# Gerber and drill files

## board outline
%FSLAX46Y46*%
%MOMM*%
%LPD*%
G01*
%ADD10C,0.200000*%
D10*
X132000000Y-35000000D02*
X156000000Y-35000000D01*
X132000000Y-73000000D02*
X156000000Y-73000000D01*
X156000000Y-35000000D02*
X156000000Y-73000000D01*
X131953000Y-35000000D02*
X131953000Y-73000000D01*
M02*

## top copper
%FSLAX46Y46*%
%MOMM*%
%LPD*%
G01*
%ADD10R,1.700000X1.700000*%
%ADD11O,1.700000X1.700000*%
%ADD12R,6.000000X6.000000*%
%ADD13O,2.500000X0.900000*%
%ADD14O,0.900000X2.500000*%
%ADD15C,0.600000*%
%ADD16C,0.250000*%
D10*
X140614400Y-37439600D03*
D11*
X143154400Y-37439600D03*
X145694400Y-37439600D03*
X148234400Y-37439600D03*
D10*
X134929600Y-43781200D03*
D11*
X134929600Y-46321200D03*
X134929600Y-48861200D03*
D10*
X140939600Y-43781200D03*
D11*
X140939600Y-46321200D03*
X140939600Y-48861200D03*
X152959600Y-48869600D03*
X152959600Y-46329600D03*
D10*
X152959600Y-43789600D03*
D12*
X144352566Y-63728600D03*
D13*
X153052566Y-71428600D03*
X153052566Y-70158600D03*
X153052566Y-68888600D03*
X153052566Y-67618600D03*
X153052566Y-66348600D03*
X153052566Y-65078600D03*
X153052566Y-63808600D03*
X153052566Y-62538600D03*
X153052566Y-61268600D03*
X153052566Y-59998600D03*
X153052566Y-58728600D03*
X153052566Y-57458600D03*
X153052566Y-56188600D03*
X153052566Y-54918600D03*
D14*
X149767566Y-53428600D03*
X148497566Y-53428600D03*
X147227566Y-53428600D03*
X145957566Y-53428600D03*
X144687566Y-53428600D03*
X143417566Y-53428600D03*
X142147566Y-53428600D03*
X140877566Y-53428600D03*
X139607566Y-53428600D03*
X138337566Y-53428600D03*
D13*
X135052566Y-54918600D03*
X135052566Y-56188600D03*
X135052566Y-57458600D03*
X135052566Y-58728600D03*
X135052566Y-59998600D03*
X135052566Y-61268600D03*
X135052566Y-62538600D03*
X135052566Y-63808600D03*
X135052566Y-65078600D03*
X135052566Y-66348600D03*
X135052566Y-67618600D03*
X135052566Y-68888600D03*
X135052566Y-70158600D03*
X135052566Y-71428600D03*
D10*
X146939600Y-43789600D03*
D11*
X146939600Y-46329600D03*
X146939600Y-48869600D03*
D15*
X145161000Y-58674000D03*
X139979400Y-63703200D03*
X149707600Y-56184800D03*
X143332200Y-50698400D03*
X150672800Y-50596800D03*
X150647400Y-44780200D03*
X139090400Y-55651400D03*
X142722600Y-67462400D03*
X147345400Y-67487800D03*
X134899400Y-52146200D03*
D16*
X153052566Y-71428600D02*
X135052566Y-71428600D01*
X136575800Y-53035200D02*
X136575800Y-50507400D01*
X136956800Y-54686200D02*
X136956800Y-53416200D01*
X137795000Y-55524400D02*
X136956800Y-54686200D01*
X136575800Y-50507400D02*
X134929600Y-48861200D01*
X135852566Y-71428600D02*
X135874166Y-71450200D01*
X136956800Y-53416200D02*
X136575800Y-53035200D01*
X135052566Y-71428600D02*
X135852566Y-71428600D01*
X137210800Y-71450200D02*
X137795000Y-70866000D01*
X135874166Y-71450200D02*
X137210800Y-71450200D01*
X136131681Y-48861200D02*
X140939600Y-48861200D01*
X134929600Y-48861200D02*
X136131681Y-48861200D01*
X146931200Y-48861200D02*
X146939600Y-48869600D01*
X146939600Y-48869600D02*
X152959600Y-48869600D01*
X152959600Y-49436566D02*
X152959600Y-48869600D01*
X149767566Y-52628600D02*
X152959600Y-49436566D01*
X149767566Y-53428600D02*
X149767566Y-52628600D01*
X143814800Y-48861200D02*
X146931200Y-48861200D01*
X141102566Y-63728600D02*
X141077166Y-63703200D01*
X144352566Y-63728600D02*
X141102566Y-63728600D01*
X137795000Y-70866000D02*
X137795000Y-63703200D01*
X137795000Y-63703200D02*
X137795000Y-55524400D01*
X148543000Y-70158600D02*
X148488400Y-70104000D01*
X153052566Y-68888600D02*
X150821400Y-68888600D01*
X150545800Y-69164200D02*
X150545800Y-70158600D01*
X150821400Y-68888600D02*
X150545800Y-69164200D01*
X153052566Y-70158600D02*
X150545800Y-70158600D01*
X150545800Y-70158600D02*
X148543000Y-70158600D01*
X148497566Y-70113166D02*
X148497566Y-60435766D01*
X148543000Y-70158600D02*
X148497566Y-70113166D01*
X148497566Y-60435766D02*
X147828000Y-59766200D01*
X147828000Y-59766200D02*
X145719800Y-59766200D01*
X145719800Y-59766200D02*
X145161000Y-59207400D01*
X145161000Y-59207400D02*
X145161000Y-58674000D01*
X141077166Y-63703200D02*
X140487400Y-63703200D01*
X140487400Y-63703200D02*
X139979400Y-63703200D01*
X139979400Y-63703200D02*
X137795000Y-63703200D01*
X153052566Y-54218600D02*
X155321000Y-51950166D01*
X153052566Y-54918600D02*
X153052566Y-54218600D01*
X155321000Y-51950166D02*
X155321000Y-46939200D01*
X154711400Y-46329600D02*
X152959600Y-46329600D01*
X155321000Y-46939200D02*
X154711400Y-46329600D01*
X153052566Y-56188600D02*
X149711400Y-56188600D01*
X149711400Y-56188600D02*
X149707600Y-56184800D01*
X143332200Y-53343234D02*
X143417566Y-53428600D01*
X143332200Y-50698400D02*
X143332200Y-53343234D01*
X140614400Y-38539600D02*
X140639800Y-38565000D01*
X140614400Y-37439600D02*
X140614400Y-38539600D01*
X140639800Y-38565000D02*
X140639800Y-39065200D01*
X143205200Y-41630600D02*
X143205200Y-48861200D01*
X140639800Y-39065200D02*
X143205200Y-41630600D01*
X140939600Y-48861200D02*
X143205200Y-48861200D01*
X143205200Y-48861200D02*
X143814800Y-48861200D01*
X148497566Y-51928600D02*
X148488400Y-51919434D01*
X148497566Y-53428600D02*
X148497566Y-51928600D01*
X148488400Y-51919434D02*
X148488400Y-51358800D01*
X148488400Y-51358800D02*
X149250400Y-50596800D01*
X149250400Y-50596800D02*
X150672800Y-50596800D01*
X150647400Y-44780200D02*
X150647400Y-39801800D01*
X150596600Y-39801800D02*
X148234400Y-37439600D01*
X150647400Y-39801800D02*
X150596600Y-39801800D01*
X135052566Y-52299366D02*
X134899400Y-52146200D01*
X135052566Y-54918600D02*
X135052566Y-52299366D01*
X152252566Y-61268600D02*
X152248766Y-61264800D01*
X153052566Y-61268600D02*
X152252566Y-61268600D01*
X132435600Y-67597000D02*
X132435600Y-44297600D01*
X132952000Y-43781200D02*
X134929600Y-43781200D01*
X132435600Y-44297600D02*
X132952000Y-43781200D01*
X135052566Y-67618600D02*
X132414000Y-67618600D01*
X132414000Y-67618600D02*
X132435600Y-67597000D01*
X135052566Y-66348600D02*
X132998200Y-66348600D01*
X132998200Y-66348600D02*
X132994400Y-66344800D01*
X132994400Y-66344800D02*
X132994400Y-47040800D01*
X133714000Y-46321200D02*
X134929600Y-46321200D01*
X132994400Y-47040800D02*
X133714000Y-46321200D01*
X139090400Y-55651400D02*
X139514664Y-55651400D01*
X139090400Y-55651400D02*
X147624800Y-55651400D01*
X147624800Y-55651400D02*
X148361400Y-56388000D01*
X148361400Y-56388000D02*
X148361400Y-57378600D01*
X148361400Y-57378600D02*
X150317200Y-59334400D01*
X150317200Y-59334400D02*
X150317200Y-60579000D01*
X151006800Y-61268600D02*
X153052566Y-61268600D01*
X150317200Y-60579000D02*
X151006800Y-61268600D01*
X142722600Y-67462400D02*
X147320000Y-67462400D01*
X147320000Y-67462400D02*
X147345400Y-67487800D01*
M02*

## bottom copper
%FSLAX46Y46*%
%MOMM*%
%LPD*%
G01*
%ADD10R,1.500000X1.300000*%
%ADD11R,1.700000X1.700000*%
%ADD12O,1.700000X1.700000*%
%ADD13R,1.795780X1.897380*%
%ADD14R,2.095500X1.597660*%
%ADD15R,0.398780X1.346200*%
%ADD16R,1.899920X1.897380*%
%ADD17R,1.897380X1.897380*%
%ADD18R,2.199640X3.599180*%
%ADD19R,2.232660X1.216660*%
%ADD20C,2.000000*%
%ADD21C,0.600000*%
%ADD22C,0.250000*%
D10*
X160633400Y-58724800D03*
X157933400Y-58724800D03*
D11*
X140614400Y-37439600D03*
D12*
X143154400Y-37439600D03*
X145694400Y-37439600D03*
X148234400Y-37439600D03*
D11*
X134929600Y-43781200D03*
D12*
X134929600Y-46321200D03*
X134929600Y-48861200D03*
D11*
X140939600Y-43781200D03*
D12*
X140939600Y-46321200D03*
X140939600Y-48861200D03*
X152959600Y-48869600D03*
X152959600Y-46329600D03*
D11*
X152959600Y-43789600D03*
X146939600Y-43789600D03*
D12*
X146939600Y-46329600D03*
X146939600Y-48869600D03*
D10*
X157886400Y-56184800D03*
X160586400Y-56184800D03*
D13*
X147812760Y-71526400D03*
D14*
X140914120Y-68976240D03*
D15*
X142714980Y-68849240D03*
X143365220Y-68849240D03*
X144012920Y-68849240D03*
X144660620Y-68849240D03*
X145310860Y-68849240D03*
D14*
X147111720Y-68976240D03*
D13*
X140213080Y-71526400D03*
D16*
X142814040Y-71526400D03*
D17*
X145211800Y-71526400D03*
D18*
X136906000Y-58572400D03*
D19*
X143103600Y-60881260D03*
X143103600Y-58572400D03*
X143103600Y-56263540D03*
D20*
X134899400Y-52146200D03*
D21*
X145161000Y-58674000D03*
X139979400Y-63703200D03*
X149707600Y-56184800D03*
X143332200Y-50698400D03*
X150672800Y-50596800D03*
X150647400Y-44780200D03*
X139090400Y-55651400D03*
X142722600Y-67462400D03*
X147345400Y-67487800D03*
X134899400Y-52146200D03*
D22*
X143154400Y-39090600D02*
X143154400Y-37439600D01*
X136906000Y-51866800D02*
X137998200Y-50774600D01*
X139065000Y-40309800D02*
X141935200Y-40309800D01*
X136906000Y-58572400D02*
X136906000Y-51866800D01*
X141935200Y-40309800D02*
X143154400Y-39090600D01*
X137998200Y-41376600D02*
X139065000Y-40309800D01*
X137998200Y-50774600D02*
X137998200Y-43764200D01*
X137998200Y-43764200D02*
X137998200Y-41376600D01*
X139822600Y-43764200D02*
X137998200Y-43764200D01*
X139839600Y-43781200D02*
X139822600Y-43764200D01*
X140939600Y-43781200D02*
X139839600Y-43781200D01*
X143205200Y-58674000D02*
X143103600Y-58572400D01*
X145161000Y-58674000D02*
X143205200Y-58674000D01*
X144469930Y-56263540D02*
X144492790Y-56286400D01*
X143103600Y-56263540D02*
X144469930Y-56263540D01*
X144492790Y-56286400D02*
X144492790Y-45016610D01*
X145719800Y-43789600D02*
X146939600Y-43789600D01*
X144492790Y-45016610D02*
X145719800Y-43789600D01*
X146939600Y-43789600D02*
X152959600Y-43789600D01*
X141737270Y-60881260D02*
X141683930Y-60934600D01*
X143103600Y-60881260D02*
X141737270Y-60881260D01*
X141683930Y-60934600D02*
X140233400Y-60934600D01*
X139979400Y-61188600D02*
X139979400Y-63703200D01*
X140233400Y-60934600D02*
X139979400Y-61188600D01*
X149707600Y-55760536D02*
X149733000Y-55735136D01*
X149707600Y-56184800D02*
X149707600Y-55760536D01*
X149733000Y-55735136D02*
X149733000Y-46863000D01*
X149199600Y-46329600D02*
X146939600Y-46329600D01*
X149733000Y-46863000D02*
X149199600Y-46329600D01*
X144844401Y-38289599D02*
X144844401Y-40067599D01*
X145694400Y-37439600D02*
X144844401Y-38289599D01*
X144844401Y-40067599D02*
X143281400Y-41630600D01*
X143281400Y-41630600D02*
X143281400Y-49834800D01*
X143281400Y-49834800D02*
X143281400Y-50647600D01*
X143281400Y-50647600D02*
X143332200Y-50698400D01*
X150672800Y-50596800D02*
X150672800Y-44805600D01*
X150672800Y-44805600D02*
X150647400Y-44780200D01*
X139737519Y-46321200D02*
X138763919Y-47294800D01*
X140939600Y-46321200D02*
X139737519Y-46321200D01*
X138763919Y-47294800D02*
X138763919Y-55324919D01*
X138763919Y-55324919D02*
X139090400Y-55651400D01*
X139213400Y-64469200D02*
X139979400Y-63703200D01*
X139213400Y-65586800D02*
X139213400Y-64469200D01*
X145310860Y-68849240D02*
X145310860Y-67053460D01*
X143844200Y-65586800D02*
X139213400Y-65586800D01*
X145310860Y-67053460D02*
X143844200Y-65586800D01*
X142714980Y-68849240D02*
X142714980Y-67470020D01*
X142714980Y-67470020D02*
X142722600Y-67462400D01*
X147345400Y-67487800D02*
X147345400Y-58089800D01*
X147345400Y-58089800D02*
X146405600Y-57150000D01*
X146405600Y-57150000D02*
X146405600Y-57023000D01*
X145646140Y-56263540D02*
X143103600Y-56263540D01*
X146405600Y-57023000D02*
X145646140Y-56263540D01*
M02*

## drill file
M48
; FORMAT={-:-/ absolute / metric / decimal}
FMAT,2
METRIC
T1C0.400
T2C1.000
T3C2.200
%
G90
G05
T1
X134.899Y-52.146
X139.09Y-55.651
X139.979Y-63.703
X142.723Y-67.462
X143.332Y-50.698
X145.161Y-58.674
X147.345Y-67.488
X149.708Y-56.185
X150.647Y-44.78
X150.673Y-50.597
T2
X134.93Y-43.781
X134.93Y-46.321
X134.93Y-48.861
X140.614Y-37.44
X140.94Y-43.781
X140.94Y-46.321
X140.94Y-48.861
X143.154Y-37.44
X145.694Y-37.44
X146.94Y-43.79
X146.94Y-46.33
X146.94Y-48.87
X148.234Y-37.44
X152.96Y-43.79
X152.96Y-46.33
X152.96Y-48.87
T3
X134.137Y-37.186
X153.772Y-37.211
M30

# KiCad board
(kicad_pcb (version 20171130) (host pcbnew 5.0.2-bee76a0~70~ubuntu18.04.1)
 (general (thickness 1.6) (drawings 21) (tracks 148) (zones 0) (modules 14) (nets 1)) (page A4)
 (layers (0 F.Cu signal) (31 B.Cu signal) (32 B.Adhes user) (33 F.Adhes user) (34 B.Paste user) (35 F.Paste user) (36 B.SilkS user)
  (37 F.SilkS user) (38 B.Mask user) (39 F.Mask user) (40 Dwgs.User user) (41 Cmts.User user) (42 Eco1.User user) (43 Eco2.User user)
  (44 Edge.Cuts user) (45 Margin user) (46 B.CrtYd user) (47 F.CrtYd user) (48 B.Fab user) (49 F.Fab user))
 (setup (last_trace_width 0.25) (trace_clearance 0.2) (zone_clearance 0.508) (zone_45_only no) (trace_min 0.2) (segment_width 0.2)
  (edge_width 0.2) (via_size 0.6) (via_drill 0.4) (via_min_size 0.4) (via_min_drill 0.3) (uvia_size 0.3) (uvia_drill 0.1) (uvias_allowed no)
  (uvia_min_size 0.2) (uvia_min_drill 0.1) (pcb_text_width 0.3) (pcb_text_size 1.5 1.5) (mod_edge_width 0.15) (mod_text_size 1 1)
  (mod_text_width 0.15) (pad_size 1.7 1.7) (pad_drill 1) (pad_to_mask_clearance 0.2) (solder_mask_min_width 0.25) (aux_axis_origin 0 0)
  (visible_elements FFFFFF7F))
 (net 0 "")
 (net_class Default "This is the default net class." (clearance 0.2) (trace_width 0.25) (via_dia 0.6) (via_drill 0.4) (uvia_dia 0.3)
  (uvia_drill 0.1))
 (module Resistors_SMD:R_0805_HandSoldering (layer B.Cu) (at 159.2834 58.7248)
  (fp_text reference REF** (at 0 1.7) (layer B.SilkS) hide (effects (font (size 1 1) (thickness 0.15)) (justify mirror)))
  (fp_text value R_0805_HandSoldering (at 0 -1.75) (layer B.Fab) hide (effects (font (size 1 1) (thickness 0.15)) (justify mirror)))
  (pad 2 smd rect (at 1.35 0) (size 1.5 1.3) (layers B.Cu B.Paste B.Mask))
  (pad 1 smd rect (at -1.35 0) (size 1.5 1.3) (layers B.Cu B.Paste B.Mask)))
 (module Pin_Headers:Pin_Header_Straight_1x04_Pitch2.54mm (layer F.Cu) (at 140.6144 37.4396 90)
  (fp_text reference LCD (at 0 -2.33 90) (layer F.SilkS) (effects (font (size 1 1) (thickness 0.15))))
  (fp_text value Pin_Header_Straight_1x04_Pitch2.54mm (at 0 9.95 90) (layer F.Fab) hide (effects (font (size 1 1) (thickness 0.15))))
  (pad GND thru_hole rect (at 0 0 90) (size 1.7 1.7) (drill 1) (layers *.Cu *.Mask))
  (pad 3.3V thru_hole oval (at 0 2.54 90) (size 1.7 1.7) (drill 1) (layers *.Cu *.Mask))
  (pad CK thru_hole oval (at 0 5.08 90) (size 1.7 1.7) (drill 1) (layers *.Cu *.Mask))
  (pad DA thru_hole oval (at 0 7.62 90) (size 1.7 1.7) (drill 1) (layers *.Cu *.Mask)))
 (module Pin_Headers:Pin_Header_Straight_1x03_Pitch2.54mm (layer F.Cu) (at 134.9296 43.7812)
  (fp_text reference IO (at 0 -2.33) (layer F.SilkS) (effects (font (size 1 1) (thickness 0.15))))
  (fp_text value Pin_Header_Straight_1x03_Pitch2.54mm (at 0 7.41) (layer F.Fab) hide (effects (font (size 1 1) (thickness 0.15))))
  (pad TX thru_hole rect (at 0 0) (size 1.7 1.7) (drill 1) (layers *.Cu *.Mask))
  (pad RX thru_hole oval (at 0 2.54) (size 1.7 1.7) (drill 1) (layers *.Cu *.Mask))
  (pad 3 thru_hole oval (at 0 5.08) (size 1.7 1.7) (drill 1) (layers *.Cu *.Mask)))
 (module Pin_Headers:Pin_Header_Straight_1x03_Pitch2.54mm (layer F.Cu) (at 140.9396 43.7812)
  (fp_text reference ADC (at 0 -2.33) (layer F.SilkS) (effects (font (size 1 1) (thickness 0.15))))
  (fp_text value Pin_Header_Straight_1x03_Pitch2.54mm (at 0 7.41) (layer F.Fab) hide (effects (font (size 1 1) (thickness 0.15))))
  (pad +3.3v thru_hole rect (at 0 0) (size 1.7 1.7) (drill 1) (layers *.Cu *.Mask))
  (pad 2 thru_hole oval (at 0 2.54) (size 1.7 1.7) (drill 1) (layers *.Cu *.Mask))
  (pad 3 thru_hole oval (at 0 5.08) (size 1.7 1.7) (drill 1) (layers *.Cu *.Mask)))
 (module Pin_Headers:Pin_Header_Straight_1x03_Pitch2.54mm (layer F.Cu) (at 152.9596 43.7896)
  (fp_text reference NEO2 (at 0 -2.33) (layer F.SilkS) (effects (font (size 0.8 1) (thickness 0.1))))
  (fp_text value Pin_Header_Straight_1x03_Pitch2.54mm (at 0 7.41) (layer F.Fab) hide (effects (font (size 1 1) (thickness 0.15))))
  (pad GND thru_hole oval (at 0 5.08) (size 1.7 1.7) (drill 1) (layers *.Cu *.Mask))
  (pad 2 thru_hole oval (at 0 2.54) (size 1.7 1.7) (drill 1) (layers *.Cu *.Mask))
  (pad +V thru_hole rect (at 0 0) (size 1.7 1.7) (drill 1) (layers *.Cu *.Mask)))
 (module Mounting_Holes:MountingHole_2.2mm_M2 (layer F.Cu) (at 134.1374 37.1856)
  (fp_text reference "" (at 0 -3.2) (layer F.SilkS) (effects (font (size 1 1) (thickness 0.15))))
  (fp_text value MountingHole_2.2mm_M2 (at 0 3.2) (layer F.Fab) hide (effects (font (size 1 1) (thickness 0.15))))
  (pad 1 np_thru_hole circle (at 0 0) (size 2.2 2.2) (drill 2.2) (layers *.Cu *.Mask F.SilkS)))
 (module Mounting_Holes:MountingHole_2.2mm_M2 (layer F.Cu) (at 153.7716 37.211)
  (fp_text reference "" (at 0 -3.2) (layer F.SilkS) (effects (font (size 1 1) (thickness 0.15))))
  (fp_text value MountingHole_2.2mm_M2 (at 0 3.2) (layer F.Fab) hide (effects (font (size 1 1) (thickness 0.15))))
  (pad 1 np_thru_hole circle (at 0 0) (size 2.2 2.2) (drill 2.2) (layers *.Cu *.Mask F.SilkS)))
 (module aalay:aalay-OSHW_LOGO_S (layer B.Cu) (at 133.9596 40.259)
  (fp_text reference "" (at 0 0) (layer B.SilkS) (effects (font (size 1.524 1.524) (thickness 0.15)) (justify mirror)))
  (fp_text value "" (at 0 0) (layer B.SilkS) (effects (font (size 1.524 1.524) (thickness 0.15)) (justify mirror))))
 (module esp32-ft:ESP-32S (layer F.Cu) (at 144 61.911262 180)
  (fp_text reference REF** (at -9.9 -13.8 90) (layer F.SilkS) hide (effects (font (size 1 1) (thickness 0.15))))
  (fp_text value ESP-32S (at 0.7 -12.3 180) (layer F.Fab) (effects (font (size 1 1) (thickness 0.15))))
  (pad 39 smd rect (at -0.352566 -1.817338) (size 6 6) (layers F.Cu F.Paste F.Mask))
  (pad 1 smd oval (at -9.052566 -9.517338) (size 2.5 0.9) (layers F.Cu F.Paste F.Mask))
  (pad 2 smd oval (at -9.052566 -8.247338) (size 2.5 0.9) (layers F.Cu F.Paste F.Mask))
  (pad 3 smd oval (at -9.052566 -6.977338) (size 2.5 0.9) (layers F.Cu F.Paste F.Mask))
  (pad 4 smd oval (at -9.052566 -5.707338) (size 2.5 0.9) (layers F.Cu F.Paste F.Mask))
  (pad 5 smd oval (at -9.052566 -4.437338) (size 2.5 0.9) (layers F.Cu F.Paste F.Mask))
  (pad 6 smd oval (at -9.052566 -3.167338) (size 2.5 0.9) (layers F.Cu F.Paste F.Mask))
  (pad 7 smd oval (at -9.052566 -1.897338) (size 2.5 0.9) (layers F.Cu F.Paste F.Mask))
  (pad 8 smd oval (at -9.052566 -0.627338) (size 2.5 0.9) (layers F.Cu F.Paste F.Mask))
  (pad 9 smd oval (at -9.052566 0.642662) (size 2.5 0.9) (layers F.Cu F.Paste F.Mask))
  (pad 10 smd oval (at -9.052566 1.912662) (size 2.5 0.9) (layers F.Cu F.Paste F.Mask))
  (pad 11 smd oval (at -9.052566 3.182662) (size 2.5 0.9) (layers F.Cu F.Paste F.Mask))
  (pad 12 smd oval (at -9.052566 4.452662) (size 2.5 0.9) (layers F.Cu F.Paste F.Mask))
  (pad 13 smd oval (at -9.052566 5.722662) (size 2.5 0.9) (layers F.Cu F.Paste F.Mask))
  (pad 14 smd oval (at -9.052566 6.992662) (size 2.5 0.9) (layers F.Cu F.Paste F.Mask))
  (pad 15 smd oval (at -5.767566 8.482662) (size 0.9 2.5) (layers F.Cu F.Paste F.Mask))
  (pad 16 smd oval (at -4.497566 8.482662) (size 0.9 2.5) (layers F.Cu F.Paste F.Mask))
  (pad 17 smd oval (at -3.227566 8.482662) (size 0.9 2.5) (layers F.Cu F.Paste F.Mask))
  (pad 18 smd oval (at -1.957566 8.482662) (size 0.9 2.5) (layers F.Cu F.Paste F.Mask))
  (pad 19 smd oval (at -0.687566 8.482662) (size 0.9 2.5) (layers F.Cu F.Paste F.Mask))
  (pad 20 smd oval (at 0.582434 8.482662) (size 0.9 2.5) (layers F.Cu F.Paste F.Mask))
  (pad 21 smd oval (at 1.852434 8.482662) (size 0.9 2.5) (layers F.Cu F.Paste F.Mask))
  (pad 22 smd oval (at 3.122434 8.482662) (size 0.9 2.5) (layers F.Cu F.Paste F.Mask))
  (pad 23 smd oval (at 4.392434 8.482662) (size 0.9 2.5) (layers F.Cu F.Paste F.Mask))
  (pad 24 smd oval (at 5.662434 8.482662) (size 0.9 2.5) (layers F.Cu F.Paste F.Mask))
  (pad 25 smd oval (at 8.947434 6.992662) (size 2.5 0.9) (layers F.Cu F.Paste F.Mask))
  (pad 26 smd oval (at 8.947434 5.722662) (size 2.5 0.9) (layers F.Cu F.Paste F.Mask))
  (pad 27 smd oval (at 8.947434 4.452662) (size 2.5 0.9) (layers F.Cu F.Paste F.Mask))
  (pad 28 smd oval (at 8.947434 3.182662) (size 2.5 0.9) (layers F.Cu F.Paste F.Mask))
  (pad 29 smd oval (at 8.947434 1.912662) (size 2.5 0.9) (layers F.Cu F.Paste F.Mask))
  (pad 30 smd oval (at 8.947434 0.642662) (size 2.5 0.9) (layers F.Cu F.Paste F.Mask))
  (pad 31 smd oval (at 8.947434 -0.627338) (size 2.5 0.9) (layers F.Cu F.Paste F.Mask))
  (pad 32 smd oval (at 8.947434 -1.897338) (size 2.5 0.9) (layers F.Cu F.Paste F.Mask))
  (pad 33 smd oval (at 8.947434 -3.167338) (size 2.5 0.9) (layers F.Cu F.Paste F.Mask))
  (pad 34 smd oval (at 8.947434 -4.437338) (size 2.5 0.9) (layers F.Cu F.Paste F.Mask))
  (pad 35 smd oval (at 8.947434 -5.707338) (size 2.5 0.9) (layers F.Cu F.Paste F.Mask))
  (pad 36 smd oval (at 8.947434 -6.977338) (size 2.5 0.9) (layers F.Cu F.Paste F.Mask))
  (pad 37 smd oval (at 8.947434 -8.247338) (size 2.5 0.9) (layers F.Cu F.Paste F.Mask))
  (pad 38 smd oval (at 8.947434 -9.517338) (size 2.5 0.9) (layers F.Cu F.Paste F.Mask)))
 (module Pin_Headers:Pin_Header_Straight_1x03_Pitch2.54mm (layer F.Cu) (at 146.9396 43.7896)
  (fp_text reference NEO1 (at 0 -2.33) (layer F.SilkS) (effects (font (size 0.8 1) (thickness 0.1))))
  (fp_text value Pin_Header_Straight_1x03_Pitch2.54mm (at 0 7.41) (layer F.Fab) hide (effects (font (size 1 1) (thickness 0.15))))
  (pad +V thru_hole rect (at 0 0) (size 1.7 1.7) (drill 1) (layers *.Cu *.Mask))
  (pad 2 thru_hole oval (at 0 2.54) (size 1.7 1.7) (drill 1) (layers *.Cu *.Mask))
  (pad GND thru_hole oval (at 0 5.08) (size 1.7 1.7) (drill 1) (layers *.Cu *.Mask)))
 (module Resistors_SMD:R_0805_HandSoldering (layer B.Cu) (at 159.2364 56.1848)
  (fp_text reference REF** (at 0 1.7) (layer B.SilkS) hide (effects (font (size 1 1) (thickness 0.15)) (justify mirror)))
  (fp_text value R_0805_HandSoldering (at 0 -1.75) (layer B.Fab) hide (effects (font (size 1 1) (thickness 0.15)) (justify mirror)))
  (pad 1 smd rect (at -1.35 0) (size 1.5 1.3) (layers B.Cu B.Paste B.Mask))
  (pad 2 smd rect (at 1.35 0) (size 1.5 1.3) (layers B.Cu B.Paste B.Mask)))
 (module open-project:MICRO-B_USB (layer B.Cu) (at 144.01292 72.9742 180)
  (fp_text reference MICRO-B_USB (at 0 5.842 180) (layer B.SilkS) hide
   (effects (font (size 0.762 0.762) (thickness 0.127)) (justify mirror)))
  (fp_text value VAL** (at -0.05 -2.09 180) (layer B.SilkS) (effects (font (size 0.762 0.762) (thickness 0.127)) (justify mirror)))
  (pad "" smd rect (at -3.79984 1.4478 180) (size 1.79578 1.89738) (layers B.Cu B.Paste B.Mask))
  (pad "" smd rect (at 3.0988 3.99796 180) (size 2.0955 1.59766) (layers B.Cu B.Paste B.Mask))
  (pad +5V smd rect (at 1.29794 4.12496 180) (size 0.39878 1.3462) (layers B.Cu B.Paste B.Mask) (clearance 0.2032))
  (pad D- smd rect (at 0.6477 4.12496 180) (size 0.39878 1.3462) (layers B.Cu B.Paste B.Mask) (clearance 0.2032))
  (pad D+ smd rect (at 0 4.12496 180) (size 0.39878 1.3462) (layers B.Cu B.Paste B.Mask) (clearance 0.2032))
  (pad ID smd rect (at -0.6477 4.12496 180) (size 0.39878 1.3462) (layers B.Cu B.Paste B.Mask) (clearance 0.2032))
  (pad GND smd rect (at -1.29794 4.12496 180) (size 0.39878 1.3462) (layers B.Cu B.Paste B.Mask) (clearance 0.2032))
  (pad "" smd rect (at -3.0988 3.99796 180) (size 2.0955 1.59766) (layers B.Cu B.Paste B.Mask))
  (pad "" smd rect (at 3.79984 1.4478 180) (size 1.79578 1.89738) (layers B.Cu B.Paste B.Mask))
  (pad "" smd rect (at 1.19888 1.4478 180) (size 1.89992 1.89738) (layers B.Cu B.Paste B.Mask))
  (pad "" smd rect (at -1.19888 1.4478 180) (size 1.89738 1.89738) (layers B.Cu B.Paste B.Mask)))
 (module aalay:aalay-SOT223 (layer B.Cu) (at 140.0048 58.5724 270)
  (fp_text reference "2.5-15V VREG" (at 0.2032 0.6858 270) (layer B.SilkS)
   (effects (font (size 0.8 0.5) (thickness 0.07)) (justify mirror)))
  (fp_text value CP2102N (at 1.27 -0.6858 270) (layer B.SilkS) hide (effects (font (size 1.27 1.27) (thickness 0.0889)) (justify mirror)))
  (pad 3.3V smd rect (at 0 3.0988 270) (size 3.59918 2.19964) (layers B.Cu B.Paste B.Mask))
  (pad GND smd rect (at 2.30886 -3.0988 270) (size 1.21666 2.23266) (layers B.Cu B.Paste B.Mask))
  (pad 3.3V smd rect (at 0 -3.0988 270) (size 1.21666 2.23266) (layers B.Cu B.Paste B.Mask))
  (pad 15V smd rect (at -2.30886 -3.0988 270) (size 1.21666 2.23266) (layers B.Cu B.Paste B.Mask)))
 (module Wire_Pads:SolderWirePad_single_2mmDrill (layer B.Cu) (at 134.8994 52.1462 270)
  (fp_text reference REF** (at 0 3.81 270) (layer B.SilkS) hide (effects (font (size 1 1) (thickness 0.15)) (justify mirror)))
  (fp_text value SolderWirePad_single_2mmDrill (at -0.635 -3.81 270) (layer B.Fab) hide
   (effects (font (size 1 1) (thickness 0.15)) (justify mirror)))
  (pad PRG smd circle (at 0 0 270) (size 2 2) (layers B.Cu B.Paste B.Mask)))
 (gr_line (start 132 35) (end 156 35) (angle 90) (layer Edge.Cuts) (width 0.2))
 (gr_line (start 132 73) (end 156 73) (angle 90) (layer Edge.Cuts) (width 0.2))
 (gr_line (start 156 35) (end 156 73) (angle 90) (layer Edge.Cuts) (width 0.2))
 (gr_line (start 131.953 35) (end 131.953 73) (angle 90) (layer Edge.Cuts) (width 0.2))
 (segment (start 153.052566 71.4286) (end 135.052566 71.4286) (width 0.25) (layer F.Cu) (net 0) (status 30))
 (segment (start 136.5758 53.0352) (end 136.5758 50.5074) (width 0.25) (layer F.Cu) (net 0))
 (segment (start 136.9568 54.6862) (end 136.9568 53.4162) (width 0.25) (layer F.Cu) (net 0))
 (segment (start 137.795 55.5244) (end 136.9568 54.6862) (width 0.25) (layer F.Cu) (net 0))
 (segment (start 136.5758 50.5074) (end 134.9296 48.8612) (width 0.25) (layer F.Cu) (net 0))
 (segment (start 135.852566 71.4286) (end 135.874166 71.4502) (width 0.25) (layer F.Cu) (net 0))
 (segment (start 136.9568 53.4162) (end 136.5758 53.0352) (width 0.25) (layer F.Cu) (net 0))
 (segment (start 135.052566 71.4286) (end 135.852566 71.4286) (width 0.25) (layer F.Cu) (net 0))
 (segment (start 137.2108 71.4502) (end 137.795 70.866) (width 0.25) (layer F.Cu) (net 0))
 (segment (start 135.874166 71.4502) (end 137.2108 71.4502) (width 0.25) (layer F.Cu) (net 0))
 (segment (start 136.131681 48.8612) (end 140.9396 48.8612) (width 0.25) (layer F.Cu) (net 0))
 (segment (start 134.9296 48.8612) (end 136.131681 48.8612) (width 0.25) (layer F.Cu) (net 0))
 (segment (start 146.9312 48.8612) (end 146.9396 48.8696) (width 0.25) (layer F.Cu) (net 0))
 (segment (start 146.9396 48.8696) (end 152.9596 48.8696) (width 0.25) (layer F.Cu) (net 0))
 (segment (start 152.9596 49.436566) (end 152.9596 48.8696) (width 0.25) (layer F.Cu) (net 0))
 (segment (start 149.767566 52.6286) (end 152.9596 49.436566) (width 0.25) (layer F.Cu) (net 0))
 (segment (start 149.767566 53.4286) (end 149.767566 52.6286) (width 0.25) (layer F.Cu) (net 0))
 (segment (start 143.8148 48.8612) (end 146.9312 48.8612) (width 0.25) (layer F.Cu) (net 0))
 (segment (start 143.1544 39.0906) (end 143.1544 37.4396) (width 0.25) (layer B.Cu) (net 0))
 (segment (start 136.906 51.8668) (end 137.9982 50.7746) (width 0.25) (layer B.Cu) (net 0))
 (segment (start 139.065 40.3098) (end 141.9352 40.3098) (width 0.25) (layer B.Cu) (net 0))
 (segment (start 136.906 58.5724) (end 136.906 51.8668) (width 0.25) (layer B.Cu) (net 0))
 (segment (start 141.9352 40.3098) (end 143.1544 39.0906) (width 0.25) (layer B.Cu) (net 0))
 (segment (start 137.9982 41.3766) (end 139.065 40.3098) (width 0.25) (layer B.Cu) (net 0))
 (segment (start 137.9982 50.7746) (end 137.9982 43.7642) (width 0.25) (layer B.Cu) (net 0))
 (segment (start 137.9982 43.7642) (end 137.9982 41.3766) (width 0.25) (layer B.Cu) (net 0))
 (segment (start 139.8226 43.7642) (end 137.9982 43.7642) (width 0.25) (layer B.Cu) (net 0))
 (segment (start 139.8396 43.7812) (end 139.8226 43.7642) (width 0.25) (layer B.Cu) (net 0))
 (segment (start 140.9396 43.7812) (end 139.8396 43.7812) (width 0.25) (layer B.Cu) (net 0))
 (segment (start 141.102566 63.7286) (end 141.077166 63.7032) (width 0.25) (layer F.Cu) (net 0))
 (segment (start 144.352566 63.7286) (end 141.102566 63.7286) (width 0.25) (layer F.Cu) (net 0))
 (segment (start 137.795 70.866) (end 137.795 63.7032) (width 0.25) (layer F.Cu) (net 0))
 (segment (start 137.795 63.7032) (end 137.795 55.5244) (width 0.25) (layer F.Cu) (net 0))
 (segment (start 148.543 70.1586) (end 148.4884 70.104) (width 0.25) (layer F.Cu) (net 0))
 (segment (start 153.052566 68.8886) (end 150.8214 68.8886) (width 0.25) (layer F.Cu) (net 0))
 (segment (start 150.5458 69.1642) (end 150.5458 70.1586) (width 0.25) (layer F.Cu) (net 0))
 (segment (start 150.8214 68.8886) (end 150.5458 69.1642) (width 0.25) (layer F.Cu) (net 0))
 (segment (start 153.052566 70.1586) (end 150.5458 70.1586) (width 0.25) (layer F.Cu) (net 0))
 (segment (start 150.5458 70.1586) (end 148.543 70.1586) (width 0.25) (layer F.Cu) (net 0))
 (segment (start 148.497566 70.113166) (end 148.497566 60.435766) (width 0.25) (layer F.Cu) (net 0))
 (segment (start 148.543 70.1586) (end 148.497566 70.113166) (width 0.25) (layer F.Cu) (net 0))
 (segment (start 148.497566 60.435766) (end 147.828 59.7662) (width 0.25) (layer F.Cu) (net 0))
 (segment (start 147.828 59.7662) (end 145.7198 59.7662) (width 0.25) (layer F.Cu) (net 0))
 (segment (start 145.7198 59.7662) (end 145.161 59.2074) (width 0.25) (layer F.Cu) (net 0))
 (segment (start 145.161 59.2074) (end 145.161 58.674) (width 0.25) (layer F.Cu) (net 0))
 (via (at 145.161 58.674) (size 0.6) (drill 0.4) (layers F.Cu B.Cu) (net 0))
 (segment (start 143.2052 58.674) (end 143.1036 58.5724) (width 0.25) (layer B.Cu) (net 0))
 (segment (start 145.161 58.674) (end 143.2052 58.674) (width 0.25) (layer B.Cu) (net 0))
 (segment (start 144.46993 56.26354) (end 144.49279 56.2864) (width 0.25) (layer B.Cu) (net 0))
 (segment (start 143.1036 56.26354) (end 144.46993 56.26354) (width 0.25) (layer B.Cu) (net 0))
 (segment (start 144.49279 56.2864) (end 144.49279 45.01661) (width 0.25) (layer B.Cu) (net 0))
 (segment (start 145.7198 43.7896) (end 146.9396 43.7896) (width 0.25) (layer B.Cu) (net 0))
 (segment (start 144.49279 45.01661) (end 145.7198 43.7896) (width 0.25) (layer B.Cu) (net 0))
 (segment (start 146.9396 43.7896) (end 152.9596 43.7896) (width 0.25) (layer B.Cu) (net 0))
 (segment (start 141.077166 63.7032) (end 140.4874 63.7032) (width 0.25) (layer F.Cu) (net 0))
 (segment (start 141.73727 60.88126) (end 141.68393 60.9346) (width 0.25) (layer B.Cu) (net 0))
 (segment (start 143.1036 60.88126) (end 141.73727 60.88126) (width 0.25) (layer B.Cu) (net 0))
 (segment (start 141.68393 60.9346) (end 140.2334 60.9346) (width 0.25) (layer B.Cu) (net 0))
 (segment (start 139.9794 61.1886) (end 139.9794 63.7032) (width 0.25) (layer B.Cu) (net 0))
 (segment (start 140.2334 60.9346) (end 139.9794 61.1886) (width 0.25) (layer B.Cu) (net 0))
 (via (at 139.9794 63.7032) (size 0.6) (drill 0.4) (layers F.Cu B.Cu) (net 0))
 (segment (start 140.4874 63.7032) (end 139.9794 63.7032) (width 0.25) (layer F.Cu) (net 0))
 (segment (start 139.9794 63.7032) (end 137.795 63.7032) (width 0.25) (layer F.Cu) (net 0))
 (segment (start 153.052566 54.2186) (end 155.321 51.950166) (width 0.25) (layer F.Cu) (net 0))
 (segment (start 153.052566 54.9186) (end 153.052566 54.2186) (width 0.25) (layer F.Cu) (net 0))
 (segment (start 155.321 51.950166) (end 155.321 46.9392) (width 0.25) (layer F.Cu) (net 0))
 (segment (start 154.7114 46.3296) (end 152.9596 46.3296) (width 0.25) (layer F.Cu) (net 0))
 (segment (start 155.321 46.9392) (end 154.7114 46.3296) (width 0.25) (layer F.Cu) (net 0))
 (via (at 149.7076 56.1848) (size 0.6) (drill 0.4) (layers F.Cu B.Cu) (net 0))
 (segment (start 153.052566 56.1886) (end 149.7114 56.1886) (width 0.25) (layer F.Cu) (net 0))
 (segment (start 149.7114 56.1886) (end 149.7076 56.1848) (width 0.25) (layer F.Cu) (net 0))
 (segment (start 149.7076 55.760536) (end 149.733 55.735136) (width 0.25) (layer B.Cu) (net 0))
 (segment (start 149.7076 56.1848) (end 149.7076 55.760536) (width 0.25) (layer B.Cu) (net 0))
 (segment (start 149.733 55.735136) (end 149.733 46.863) (width 0.25) (layer B.Cu) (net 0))
 (segment (start 149.1996 46.3296) (end 146.9396 46.3296) (width 0.25) (layer B.Cu) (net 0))
 (segment (start 149.733 46.863) (end 149.1996 46.3296) (width 0.25) (layer B.Cu) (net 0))
 (segment (start 144.844401 38.289599) (end 144.844401 40.067599) (width 0.25) (layer B.Cu) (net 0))
 (segment (start 145.6944 37.4396) (end 144.844401 38.289599) (width 0.25) (layer B.Cu) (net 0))
 (segment (start 144.844401 40.067599) (end 143.2814 41.6306) (width 0.25) (layer B.Cu) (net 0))
 (segment (start 143.2814 41.6306) (end 143.2814 49.8348) (width 0.25) (layer B.Cu) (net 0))
 (segment (start 143.2814 49.8348) (end 143.2814 50.6476) (width 0.25) (layer B.Cu) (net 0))
 (via (at 143.3322 50.6984) (size 0.6) (drill 0.4) (layers F.Cu B.Cu) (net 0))
 (segment (start 143.2814 50.6476) (end 143.3322 50.6984) (width 0.25) (layer B.Cu) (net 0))
 (segment (start 143.3322 53.343234) (end 143.417566 53.4286) (width 0.25) (layer F.Cu) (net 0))
 (segment (start 143.3322 50.6984) (end 143.3322 53.343234) (width 0.25) (layer F.Cu) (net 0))
 (segment (start 140.6144 38.5396) (end 140.6398 38.565) (width 0.25) (layer F.Cu) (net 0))
 (segment (start 140.6144 37.4396) (end 140.6144 38.5396) (width 0.25) (layer F.Cu) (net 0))
 (segment (start 140.6398 38.565) (end 140.6398 39.0652) (width 0.25) (layer F.Cu) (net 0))
 (segment (start 143.2052 41.6306) (end 143.2052 48.8612) (width 0.25) (layer F.Cu) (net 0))
 (segment (start 140.6398 39.0652) (end 143.2052 41.6306) (width 0.25) (layer F.Cu) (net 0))
 (segment (start 140.9396 48.8612) (end 143.2052 48.8612) (width 0.25) (layer F.Cu) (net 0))
 (segment (start 143.2052 48.8612) (end 143.8148 48.8612) (width 0.25) (layer F.Cu) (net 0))
 (segment (start 148.497566 51.9286) (end 148.4884 51.919434) (width 0.25) (layer F.Cu) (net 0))
 (segment (start 148.497566 53.4286) (end 148.497566 51.9286) (width 0.25) (layer F.Cu) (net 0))
 (segment (start 148.4884 51.919434) (end 148.4884 51.3588) (width 0.25) (layer F.Cu) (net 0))
 (via (at 150.6728 50.5968) (size 0.6) (drill 0.4) (layers F.Cu B.Cu) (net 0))
 (segment (start 148.4884 51.3588) (end 149.2504 50.5968) (width 0.25) (layer F.Cu) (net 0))
 (segment (start 149.2504 50.5968) (end 150.6728 50.5968) (width 0.25) (layer F.Cu) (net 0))
 (via (at 150.6474 44.7802) (size 0.6) (drill 0.4) (layers F.Cu B.Cu) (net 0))
 (segment (start 150.6728 50.5968) (end 150.6728 44.8056) (width 0.25) (layer B.Cu) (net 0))
 (segment (start 150.6728 44.8056) (end 150.6474 44.7802) (width 0.25) (layer B.Cu) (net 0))
 (segment (start 150.6474 44.7802) (end 150.6474 39.8018) (width 0.25) (layer F.Cu) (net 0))
 (segment (start 150.5966 39.8018) (end 148.2344 37.4396) (width 0.25) (layer F.Cu) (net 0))
 (segment (start 150.6474 39.8018) (end 150.5966 39.8018) (width 0.25) (layer F.Cu) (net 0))
 (segment (start 135.052566 52.299366) (end 134.8994 52.1462) (width 0.25) (layer F.Cu) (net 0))
 (segment (start 135.052566 54.9186) (end 135.052566 52.299366) (width 0.25) (layer F.Cu) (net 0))
 (segment (start 152.252566 61.2686) (end 152.248766 61.2648) (width 0.25) (layer F.Cu) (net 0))
 (segment (start 153.052566 61.2686) (end 152.252566 61.2686) (width 0.25) (layer F.Cu) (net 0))
 (segment (start 132.4356 67.597) (end 132.4356 44.2976) (width 0.25) (layer F.Cu) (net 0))
 (segment (start 132.952 43.7812) (end 134.9296 43.7812) (width 0.25) (layer F.Cu) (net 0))
 (segment (start 132.4356 44.2976) (end 132.952 43.7812) (width 0.25) (layer F.Cu) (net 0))
 (segment (start 135.052566 67.6186) (end 132.414 67.6186) (width 0.25) (layer F.Cu) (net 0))
 (segment (start 132.414 67.6186) (end 132.4356 67.597) (width 0.25) (layer F.Cu) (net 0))
 (segment (start 135.052566 66.3486) (end 132.9982 66.3486) (width 0.25) (layer F.Cu) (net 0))
 (segment (start 132.9982 66.3486) (end 132.9944 66.3448) (width 0.25) (layer F.Cu) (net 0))
 (segment (start 132.9944 66.3448) (end 132.9944 47.0408) (width 0.25) (layer F.Cu) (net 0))
 (segment (start 133.714 46.3212) (end 134.9296 46.3212) (width 0.25) (layer F.Cu) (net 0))
 (segment (start 132.9944 47.0408) (end 133.714 46.3212) (width 0.25) (layer F.Cu) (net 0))
 (segment (start 139.737519 46.3212) (end 138.763919 47.2948) (width 0.25) (layer B.Cu) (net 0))
 (segment (start 140.9396 46.3212) (end 139.737519 46.3212) (width 0.25) (layer B.Cu) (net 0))
 (via (at 139.0904 55.6514) (size 0.6) (drill 0.4) (layers F.Cu B.Cu) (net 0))
 (segment (start 138.763919 47.2948) (end 138.763919 55.324919) (width 0.25) (layer B.Cu) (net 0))
 (segment (start 138.763919 55.324919) (end 139.0904 55.6514) (width 0.25) (layer B.Cu) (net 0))
 (segment (start 139.0904 55.6514) (end 139.514664 55.6514) (width 0.25) (layer F.Cu) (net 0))
 (segment (start 139.2134 64.4692) (end 139.9794 63.7032) (width 0.25) (layer B.Cu) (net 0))
 (segment (start 139.2134 65.5868) (end 139.2134 64.4692) (width 0.25) (layer B.Cu) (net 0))
 (segment (start 145.31086 68.84924) (end 145.31086 67.05346) (width 0.25) (layer B.Cu) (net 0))
 (segment (start 143.8442 65.5868) (end 139.2134 65.5868) (width 0.25) (layer B.Cu) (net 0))
 (segment (start 145.31086 67.05346) (end 143.8442 65.5868) (width 0.25) (layer B.Cu) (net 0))
 (segment (start 139.0904 55.6514) (end 147.6248 55.6514) (width 0.25) (layer F.Cu) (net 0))
 (segment (start 147.6248 55.6514) (end 148.3614 56.388) (width 0.25) (layer F.Cu) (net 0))
 (segment (start 148.3614 56.388) (end 148.3614 57.3786) (width 0.25) (layer F.Cu) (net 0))
 (segment (start 148.3614 57.3786) (end 150.3172 59.3344) (width 0.25) (layer F.Cu) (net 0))
 (segment (start 150.3172 59.3344) (end 150.3172 60.579) (width 0.25) (layer F.Cu) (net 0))
 (segment (start 151.0068 61.2686) (end 153.052566 61.2686) (width 0.25) (layer F.Cu) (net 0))
 (segment (start 150.3172 60.579) (end 151.0068 61.2686) (width 0.25) (layer F.Cu) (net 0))
 (segment (start 142.71498 68.84924) (end 142.71498 67.47002) (width 0.25) (layer B.Cu) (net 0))
 (via (at 142.7226 67.4624) (size 0.6) (drill 0.4) (layers F.Cu B.Cu) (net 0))
 (segment (start 142.71498 67.47002) (end 142.7226 67.4624) (width 0.25) (layer B.Cu) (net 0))
 (via (at 147.3454 67.4878) (size 0.6) (drill 0.4) (layers F.Cu B.Cu) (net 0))
 (segment (start 142.7226 67.4624) (end 147.32 67.4624) (width 0.25) (layer F.Cu) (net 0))
 (segment (start 147.32 67.4624) (end 147.3454 67.4878) (width 0.25) (layer F.Cu) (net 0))
 (segment (start 147.3454 67.4878) (end 147.3454 58.0898) (width 0.25) (layer B.Cu) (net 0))
 (segment (start 147.3454 58.0898) (end 146.4056 57.15) (width 0.25) (layer B.Cu) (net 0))
 (segment (start 146.4056 57.15) (end 146.4056 57.023) (width 0.25) (layer B.Cu) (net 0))
 (segment (start 145.64614 56.26354) (end 143.1036 56.26354) (width 0.25) (layer B.Cu) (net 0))
 (segment (start 146.4056 57.023) (end 145.64614 56.26354) (width 0.25) (layer B.Cu) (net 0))
 (via (at 134.8994 52.1462) (size 0.6) (drill 0.4) (layers F.Cu B.Cu) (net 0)))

